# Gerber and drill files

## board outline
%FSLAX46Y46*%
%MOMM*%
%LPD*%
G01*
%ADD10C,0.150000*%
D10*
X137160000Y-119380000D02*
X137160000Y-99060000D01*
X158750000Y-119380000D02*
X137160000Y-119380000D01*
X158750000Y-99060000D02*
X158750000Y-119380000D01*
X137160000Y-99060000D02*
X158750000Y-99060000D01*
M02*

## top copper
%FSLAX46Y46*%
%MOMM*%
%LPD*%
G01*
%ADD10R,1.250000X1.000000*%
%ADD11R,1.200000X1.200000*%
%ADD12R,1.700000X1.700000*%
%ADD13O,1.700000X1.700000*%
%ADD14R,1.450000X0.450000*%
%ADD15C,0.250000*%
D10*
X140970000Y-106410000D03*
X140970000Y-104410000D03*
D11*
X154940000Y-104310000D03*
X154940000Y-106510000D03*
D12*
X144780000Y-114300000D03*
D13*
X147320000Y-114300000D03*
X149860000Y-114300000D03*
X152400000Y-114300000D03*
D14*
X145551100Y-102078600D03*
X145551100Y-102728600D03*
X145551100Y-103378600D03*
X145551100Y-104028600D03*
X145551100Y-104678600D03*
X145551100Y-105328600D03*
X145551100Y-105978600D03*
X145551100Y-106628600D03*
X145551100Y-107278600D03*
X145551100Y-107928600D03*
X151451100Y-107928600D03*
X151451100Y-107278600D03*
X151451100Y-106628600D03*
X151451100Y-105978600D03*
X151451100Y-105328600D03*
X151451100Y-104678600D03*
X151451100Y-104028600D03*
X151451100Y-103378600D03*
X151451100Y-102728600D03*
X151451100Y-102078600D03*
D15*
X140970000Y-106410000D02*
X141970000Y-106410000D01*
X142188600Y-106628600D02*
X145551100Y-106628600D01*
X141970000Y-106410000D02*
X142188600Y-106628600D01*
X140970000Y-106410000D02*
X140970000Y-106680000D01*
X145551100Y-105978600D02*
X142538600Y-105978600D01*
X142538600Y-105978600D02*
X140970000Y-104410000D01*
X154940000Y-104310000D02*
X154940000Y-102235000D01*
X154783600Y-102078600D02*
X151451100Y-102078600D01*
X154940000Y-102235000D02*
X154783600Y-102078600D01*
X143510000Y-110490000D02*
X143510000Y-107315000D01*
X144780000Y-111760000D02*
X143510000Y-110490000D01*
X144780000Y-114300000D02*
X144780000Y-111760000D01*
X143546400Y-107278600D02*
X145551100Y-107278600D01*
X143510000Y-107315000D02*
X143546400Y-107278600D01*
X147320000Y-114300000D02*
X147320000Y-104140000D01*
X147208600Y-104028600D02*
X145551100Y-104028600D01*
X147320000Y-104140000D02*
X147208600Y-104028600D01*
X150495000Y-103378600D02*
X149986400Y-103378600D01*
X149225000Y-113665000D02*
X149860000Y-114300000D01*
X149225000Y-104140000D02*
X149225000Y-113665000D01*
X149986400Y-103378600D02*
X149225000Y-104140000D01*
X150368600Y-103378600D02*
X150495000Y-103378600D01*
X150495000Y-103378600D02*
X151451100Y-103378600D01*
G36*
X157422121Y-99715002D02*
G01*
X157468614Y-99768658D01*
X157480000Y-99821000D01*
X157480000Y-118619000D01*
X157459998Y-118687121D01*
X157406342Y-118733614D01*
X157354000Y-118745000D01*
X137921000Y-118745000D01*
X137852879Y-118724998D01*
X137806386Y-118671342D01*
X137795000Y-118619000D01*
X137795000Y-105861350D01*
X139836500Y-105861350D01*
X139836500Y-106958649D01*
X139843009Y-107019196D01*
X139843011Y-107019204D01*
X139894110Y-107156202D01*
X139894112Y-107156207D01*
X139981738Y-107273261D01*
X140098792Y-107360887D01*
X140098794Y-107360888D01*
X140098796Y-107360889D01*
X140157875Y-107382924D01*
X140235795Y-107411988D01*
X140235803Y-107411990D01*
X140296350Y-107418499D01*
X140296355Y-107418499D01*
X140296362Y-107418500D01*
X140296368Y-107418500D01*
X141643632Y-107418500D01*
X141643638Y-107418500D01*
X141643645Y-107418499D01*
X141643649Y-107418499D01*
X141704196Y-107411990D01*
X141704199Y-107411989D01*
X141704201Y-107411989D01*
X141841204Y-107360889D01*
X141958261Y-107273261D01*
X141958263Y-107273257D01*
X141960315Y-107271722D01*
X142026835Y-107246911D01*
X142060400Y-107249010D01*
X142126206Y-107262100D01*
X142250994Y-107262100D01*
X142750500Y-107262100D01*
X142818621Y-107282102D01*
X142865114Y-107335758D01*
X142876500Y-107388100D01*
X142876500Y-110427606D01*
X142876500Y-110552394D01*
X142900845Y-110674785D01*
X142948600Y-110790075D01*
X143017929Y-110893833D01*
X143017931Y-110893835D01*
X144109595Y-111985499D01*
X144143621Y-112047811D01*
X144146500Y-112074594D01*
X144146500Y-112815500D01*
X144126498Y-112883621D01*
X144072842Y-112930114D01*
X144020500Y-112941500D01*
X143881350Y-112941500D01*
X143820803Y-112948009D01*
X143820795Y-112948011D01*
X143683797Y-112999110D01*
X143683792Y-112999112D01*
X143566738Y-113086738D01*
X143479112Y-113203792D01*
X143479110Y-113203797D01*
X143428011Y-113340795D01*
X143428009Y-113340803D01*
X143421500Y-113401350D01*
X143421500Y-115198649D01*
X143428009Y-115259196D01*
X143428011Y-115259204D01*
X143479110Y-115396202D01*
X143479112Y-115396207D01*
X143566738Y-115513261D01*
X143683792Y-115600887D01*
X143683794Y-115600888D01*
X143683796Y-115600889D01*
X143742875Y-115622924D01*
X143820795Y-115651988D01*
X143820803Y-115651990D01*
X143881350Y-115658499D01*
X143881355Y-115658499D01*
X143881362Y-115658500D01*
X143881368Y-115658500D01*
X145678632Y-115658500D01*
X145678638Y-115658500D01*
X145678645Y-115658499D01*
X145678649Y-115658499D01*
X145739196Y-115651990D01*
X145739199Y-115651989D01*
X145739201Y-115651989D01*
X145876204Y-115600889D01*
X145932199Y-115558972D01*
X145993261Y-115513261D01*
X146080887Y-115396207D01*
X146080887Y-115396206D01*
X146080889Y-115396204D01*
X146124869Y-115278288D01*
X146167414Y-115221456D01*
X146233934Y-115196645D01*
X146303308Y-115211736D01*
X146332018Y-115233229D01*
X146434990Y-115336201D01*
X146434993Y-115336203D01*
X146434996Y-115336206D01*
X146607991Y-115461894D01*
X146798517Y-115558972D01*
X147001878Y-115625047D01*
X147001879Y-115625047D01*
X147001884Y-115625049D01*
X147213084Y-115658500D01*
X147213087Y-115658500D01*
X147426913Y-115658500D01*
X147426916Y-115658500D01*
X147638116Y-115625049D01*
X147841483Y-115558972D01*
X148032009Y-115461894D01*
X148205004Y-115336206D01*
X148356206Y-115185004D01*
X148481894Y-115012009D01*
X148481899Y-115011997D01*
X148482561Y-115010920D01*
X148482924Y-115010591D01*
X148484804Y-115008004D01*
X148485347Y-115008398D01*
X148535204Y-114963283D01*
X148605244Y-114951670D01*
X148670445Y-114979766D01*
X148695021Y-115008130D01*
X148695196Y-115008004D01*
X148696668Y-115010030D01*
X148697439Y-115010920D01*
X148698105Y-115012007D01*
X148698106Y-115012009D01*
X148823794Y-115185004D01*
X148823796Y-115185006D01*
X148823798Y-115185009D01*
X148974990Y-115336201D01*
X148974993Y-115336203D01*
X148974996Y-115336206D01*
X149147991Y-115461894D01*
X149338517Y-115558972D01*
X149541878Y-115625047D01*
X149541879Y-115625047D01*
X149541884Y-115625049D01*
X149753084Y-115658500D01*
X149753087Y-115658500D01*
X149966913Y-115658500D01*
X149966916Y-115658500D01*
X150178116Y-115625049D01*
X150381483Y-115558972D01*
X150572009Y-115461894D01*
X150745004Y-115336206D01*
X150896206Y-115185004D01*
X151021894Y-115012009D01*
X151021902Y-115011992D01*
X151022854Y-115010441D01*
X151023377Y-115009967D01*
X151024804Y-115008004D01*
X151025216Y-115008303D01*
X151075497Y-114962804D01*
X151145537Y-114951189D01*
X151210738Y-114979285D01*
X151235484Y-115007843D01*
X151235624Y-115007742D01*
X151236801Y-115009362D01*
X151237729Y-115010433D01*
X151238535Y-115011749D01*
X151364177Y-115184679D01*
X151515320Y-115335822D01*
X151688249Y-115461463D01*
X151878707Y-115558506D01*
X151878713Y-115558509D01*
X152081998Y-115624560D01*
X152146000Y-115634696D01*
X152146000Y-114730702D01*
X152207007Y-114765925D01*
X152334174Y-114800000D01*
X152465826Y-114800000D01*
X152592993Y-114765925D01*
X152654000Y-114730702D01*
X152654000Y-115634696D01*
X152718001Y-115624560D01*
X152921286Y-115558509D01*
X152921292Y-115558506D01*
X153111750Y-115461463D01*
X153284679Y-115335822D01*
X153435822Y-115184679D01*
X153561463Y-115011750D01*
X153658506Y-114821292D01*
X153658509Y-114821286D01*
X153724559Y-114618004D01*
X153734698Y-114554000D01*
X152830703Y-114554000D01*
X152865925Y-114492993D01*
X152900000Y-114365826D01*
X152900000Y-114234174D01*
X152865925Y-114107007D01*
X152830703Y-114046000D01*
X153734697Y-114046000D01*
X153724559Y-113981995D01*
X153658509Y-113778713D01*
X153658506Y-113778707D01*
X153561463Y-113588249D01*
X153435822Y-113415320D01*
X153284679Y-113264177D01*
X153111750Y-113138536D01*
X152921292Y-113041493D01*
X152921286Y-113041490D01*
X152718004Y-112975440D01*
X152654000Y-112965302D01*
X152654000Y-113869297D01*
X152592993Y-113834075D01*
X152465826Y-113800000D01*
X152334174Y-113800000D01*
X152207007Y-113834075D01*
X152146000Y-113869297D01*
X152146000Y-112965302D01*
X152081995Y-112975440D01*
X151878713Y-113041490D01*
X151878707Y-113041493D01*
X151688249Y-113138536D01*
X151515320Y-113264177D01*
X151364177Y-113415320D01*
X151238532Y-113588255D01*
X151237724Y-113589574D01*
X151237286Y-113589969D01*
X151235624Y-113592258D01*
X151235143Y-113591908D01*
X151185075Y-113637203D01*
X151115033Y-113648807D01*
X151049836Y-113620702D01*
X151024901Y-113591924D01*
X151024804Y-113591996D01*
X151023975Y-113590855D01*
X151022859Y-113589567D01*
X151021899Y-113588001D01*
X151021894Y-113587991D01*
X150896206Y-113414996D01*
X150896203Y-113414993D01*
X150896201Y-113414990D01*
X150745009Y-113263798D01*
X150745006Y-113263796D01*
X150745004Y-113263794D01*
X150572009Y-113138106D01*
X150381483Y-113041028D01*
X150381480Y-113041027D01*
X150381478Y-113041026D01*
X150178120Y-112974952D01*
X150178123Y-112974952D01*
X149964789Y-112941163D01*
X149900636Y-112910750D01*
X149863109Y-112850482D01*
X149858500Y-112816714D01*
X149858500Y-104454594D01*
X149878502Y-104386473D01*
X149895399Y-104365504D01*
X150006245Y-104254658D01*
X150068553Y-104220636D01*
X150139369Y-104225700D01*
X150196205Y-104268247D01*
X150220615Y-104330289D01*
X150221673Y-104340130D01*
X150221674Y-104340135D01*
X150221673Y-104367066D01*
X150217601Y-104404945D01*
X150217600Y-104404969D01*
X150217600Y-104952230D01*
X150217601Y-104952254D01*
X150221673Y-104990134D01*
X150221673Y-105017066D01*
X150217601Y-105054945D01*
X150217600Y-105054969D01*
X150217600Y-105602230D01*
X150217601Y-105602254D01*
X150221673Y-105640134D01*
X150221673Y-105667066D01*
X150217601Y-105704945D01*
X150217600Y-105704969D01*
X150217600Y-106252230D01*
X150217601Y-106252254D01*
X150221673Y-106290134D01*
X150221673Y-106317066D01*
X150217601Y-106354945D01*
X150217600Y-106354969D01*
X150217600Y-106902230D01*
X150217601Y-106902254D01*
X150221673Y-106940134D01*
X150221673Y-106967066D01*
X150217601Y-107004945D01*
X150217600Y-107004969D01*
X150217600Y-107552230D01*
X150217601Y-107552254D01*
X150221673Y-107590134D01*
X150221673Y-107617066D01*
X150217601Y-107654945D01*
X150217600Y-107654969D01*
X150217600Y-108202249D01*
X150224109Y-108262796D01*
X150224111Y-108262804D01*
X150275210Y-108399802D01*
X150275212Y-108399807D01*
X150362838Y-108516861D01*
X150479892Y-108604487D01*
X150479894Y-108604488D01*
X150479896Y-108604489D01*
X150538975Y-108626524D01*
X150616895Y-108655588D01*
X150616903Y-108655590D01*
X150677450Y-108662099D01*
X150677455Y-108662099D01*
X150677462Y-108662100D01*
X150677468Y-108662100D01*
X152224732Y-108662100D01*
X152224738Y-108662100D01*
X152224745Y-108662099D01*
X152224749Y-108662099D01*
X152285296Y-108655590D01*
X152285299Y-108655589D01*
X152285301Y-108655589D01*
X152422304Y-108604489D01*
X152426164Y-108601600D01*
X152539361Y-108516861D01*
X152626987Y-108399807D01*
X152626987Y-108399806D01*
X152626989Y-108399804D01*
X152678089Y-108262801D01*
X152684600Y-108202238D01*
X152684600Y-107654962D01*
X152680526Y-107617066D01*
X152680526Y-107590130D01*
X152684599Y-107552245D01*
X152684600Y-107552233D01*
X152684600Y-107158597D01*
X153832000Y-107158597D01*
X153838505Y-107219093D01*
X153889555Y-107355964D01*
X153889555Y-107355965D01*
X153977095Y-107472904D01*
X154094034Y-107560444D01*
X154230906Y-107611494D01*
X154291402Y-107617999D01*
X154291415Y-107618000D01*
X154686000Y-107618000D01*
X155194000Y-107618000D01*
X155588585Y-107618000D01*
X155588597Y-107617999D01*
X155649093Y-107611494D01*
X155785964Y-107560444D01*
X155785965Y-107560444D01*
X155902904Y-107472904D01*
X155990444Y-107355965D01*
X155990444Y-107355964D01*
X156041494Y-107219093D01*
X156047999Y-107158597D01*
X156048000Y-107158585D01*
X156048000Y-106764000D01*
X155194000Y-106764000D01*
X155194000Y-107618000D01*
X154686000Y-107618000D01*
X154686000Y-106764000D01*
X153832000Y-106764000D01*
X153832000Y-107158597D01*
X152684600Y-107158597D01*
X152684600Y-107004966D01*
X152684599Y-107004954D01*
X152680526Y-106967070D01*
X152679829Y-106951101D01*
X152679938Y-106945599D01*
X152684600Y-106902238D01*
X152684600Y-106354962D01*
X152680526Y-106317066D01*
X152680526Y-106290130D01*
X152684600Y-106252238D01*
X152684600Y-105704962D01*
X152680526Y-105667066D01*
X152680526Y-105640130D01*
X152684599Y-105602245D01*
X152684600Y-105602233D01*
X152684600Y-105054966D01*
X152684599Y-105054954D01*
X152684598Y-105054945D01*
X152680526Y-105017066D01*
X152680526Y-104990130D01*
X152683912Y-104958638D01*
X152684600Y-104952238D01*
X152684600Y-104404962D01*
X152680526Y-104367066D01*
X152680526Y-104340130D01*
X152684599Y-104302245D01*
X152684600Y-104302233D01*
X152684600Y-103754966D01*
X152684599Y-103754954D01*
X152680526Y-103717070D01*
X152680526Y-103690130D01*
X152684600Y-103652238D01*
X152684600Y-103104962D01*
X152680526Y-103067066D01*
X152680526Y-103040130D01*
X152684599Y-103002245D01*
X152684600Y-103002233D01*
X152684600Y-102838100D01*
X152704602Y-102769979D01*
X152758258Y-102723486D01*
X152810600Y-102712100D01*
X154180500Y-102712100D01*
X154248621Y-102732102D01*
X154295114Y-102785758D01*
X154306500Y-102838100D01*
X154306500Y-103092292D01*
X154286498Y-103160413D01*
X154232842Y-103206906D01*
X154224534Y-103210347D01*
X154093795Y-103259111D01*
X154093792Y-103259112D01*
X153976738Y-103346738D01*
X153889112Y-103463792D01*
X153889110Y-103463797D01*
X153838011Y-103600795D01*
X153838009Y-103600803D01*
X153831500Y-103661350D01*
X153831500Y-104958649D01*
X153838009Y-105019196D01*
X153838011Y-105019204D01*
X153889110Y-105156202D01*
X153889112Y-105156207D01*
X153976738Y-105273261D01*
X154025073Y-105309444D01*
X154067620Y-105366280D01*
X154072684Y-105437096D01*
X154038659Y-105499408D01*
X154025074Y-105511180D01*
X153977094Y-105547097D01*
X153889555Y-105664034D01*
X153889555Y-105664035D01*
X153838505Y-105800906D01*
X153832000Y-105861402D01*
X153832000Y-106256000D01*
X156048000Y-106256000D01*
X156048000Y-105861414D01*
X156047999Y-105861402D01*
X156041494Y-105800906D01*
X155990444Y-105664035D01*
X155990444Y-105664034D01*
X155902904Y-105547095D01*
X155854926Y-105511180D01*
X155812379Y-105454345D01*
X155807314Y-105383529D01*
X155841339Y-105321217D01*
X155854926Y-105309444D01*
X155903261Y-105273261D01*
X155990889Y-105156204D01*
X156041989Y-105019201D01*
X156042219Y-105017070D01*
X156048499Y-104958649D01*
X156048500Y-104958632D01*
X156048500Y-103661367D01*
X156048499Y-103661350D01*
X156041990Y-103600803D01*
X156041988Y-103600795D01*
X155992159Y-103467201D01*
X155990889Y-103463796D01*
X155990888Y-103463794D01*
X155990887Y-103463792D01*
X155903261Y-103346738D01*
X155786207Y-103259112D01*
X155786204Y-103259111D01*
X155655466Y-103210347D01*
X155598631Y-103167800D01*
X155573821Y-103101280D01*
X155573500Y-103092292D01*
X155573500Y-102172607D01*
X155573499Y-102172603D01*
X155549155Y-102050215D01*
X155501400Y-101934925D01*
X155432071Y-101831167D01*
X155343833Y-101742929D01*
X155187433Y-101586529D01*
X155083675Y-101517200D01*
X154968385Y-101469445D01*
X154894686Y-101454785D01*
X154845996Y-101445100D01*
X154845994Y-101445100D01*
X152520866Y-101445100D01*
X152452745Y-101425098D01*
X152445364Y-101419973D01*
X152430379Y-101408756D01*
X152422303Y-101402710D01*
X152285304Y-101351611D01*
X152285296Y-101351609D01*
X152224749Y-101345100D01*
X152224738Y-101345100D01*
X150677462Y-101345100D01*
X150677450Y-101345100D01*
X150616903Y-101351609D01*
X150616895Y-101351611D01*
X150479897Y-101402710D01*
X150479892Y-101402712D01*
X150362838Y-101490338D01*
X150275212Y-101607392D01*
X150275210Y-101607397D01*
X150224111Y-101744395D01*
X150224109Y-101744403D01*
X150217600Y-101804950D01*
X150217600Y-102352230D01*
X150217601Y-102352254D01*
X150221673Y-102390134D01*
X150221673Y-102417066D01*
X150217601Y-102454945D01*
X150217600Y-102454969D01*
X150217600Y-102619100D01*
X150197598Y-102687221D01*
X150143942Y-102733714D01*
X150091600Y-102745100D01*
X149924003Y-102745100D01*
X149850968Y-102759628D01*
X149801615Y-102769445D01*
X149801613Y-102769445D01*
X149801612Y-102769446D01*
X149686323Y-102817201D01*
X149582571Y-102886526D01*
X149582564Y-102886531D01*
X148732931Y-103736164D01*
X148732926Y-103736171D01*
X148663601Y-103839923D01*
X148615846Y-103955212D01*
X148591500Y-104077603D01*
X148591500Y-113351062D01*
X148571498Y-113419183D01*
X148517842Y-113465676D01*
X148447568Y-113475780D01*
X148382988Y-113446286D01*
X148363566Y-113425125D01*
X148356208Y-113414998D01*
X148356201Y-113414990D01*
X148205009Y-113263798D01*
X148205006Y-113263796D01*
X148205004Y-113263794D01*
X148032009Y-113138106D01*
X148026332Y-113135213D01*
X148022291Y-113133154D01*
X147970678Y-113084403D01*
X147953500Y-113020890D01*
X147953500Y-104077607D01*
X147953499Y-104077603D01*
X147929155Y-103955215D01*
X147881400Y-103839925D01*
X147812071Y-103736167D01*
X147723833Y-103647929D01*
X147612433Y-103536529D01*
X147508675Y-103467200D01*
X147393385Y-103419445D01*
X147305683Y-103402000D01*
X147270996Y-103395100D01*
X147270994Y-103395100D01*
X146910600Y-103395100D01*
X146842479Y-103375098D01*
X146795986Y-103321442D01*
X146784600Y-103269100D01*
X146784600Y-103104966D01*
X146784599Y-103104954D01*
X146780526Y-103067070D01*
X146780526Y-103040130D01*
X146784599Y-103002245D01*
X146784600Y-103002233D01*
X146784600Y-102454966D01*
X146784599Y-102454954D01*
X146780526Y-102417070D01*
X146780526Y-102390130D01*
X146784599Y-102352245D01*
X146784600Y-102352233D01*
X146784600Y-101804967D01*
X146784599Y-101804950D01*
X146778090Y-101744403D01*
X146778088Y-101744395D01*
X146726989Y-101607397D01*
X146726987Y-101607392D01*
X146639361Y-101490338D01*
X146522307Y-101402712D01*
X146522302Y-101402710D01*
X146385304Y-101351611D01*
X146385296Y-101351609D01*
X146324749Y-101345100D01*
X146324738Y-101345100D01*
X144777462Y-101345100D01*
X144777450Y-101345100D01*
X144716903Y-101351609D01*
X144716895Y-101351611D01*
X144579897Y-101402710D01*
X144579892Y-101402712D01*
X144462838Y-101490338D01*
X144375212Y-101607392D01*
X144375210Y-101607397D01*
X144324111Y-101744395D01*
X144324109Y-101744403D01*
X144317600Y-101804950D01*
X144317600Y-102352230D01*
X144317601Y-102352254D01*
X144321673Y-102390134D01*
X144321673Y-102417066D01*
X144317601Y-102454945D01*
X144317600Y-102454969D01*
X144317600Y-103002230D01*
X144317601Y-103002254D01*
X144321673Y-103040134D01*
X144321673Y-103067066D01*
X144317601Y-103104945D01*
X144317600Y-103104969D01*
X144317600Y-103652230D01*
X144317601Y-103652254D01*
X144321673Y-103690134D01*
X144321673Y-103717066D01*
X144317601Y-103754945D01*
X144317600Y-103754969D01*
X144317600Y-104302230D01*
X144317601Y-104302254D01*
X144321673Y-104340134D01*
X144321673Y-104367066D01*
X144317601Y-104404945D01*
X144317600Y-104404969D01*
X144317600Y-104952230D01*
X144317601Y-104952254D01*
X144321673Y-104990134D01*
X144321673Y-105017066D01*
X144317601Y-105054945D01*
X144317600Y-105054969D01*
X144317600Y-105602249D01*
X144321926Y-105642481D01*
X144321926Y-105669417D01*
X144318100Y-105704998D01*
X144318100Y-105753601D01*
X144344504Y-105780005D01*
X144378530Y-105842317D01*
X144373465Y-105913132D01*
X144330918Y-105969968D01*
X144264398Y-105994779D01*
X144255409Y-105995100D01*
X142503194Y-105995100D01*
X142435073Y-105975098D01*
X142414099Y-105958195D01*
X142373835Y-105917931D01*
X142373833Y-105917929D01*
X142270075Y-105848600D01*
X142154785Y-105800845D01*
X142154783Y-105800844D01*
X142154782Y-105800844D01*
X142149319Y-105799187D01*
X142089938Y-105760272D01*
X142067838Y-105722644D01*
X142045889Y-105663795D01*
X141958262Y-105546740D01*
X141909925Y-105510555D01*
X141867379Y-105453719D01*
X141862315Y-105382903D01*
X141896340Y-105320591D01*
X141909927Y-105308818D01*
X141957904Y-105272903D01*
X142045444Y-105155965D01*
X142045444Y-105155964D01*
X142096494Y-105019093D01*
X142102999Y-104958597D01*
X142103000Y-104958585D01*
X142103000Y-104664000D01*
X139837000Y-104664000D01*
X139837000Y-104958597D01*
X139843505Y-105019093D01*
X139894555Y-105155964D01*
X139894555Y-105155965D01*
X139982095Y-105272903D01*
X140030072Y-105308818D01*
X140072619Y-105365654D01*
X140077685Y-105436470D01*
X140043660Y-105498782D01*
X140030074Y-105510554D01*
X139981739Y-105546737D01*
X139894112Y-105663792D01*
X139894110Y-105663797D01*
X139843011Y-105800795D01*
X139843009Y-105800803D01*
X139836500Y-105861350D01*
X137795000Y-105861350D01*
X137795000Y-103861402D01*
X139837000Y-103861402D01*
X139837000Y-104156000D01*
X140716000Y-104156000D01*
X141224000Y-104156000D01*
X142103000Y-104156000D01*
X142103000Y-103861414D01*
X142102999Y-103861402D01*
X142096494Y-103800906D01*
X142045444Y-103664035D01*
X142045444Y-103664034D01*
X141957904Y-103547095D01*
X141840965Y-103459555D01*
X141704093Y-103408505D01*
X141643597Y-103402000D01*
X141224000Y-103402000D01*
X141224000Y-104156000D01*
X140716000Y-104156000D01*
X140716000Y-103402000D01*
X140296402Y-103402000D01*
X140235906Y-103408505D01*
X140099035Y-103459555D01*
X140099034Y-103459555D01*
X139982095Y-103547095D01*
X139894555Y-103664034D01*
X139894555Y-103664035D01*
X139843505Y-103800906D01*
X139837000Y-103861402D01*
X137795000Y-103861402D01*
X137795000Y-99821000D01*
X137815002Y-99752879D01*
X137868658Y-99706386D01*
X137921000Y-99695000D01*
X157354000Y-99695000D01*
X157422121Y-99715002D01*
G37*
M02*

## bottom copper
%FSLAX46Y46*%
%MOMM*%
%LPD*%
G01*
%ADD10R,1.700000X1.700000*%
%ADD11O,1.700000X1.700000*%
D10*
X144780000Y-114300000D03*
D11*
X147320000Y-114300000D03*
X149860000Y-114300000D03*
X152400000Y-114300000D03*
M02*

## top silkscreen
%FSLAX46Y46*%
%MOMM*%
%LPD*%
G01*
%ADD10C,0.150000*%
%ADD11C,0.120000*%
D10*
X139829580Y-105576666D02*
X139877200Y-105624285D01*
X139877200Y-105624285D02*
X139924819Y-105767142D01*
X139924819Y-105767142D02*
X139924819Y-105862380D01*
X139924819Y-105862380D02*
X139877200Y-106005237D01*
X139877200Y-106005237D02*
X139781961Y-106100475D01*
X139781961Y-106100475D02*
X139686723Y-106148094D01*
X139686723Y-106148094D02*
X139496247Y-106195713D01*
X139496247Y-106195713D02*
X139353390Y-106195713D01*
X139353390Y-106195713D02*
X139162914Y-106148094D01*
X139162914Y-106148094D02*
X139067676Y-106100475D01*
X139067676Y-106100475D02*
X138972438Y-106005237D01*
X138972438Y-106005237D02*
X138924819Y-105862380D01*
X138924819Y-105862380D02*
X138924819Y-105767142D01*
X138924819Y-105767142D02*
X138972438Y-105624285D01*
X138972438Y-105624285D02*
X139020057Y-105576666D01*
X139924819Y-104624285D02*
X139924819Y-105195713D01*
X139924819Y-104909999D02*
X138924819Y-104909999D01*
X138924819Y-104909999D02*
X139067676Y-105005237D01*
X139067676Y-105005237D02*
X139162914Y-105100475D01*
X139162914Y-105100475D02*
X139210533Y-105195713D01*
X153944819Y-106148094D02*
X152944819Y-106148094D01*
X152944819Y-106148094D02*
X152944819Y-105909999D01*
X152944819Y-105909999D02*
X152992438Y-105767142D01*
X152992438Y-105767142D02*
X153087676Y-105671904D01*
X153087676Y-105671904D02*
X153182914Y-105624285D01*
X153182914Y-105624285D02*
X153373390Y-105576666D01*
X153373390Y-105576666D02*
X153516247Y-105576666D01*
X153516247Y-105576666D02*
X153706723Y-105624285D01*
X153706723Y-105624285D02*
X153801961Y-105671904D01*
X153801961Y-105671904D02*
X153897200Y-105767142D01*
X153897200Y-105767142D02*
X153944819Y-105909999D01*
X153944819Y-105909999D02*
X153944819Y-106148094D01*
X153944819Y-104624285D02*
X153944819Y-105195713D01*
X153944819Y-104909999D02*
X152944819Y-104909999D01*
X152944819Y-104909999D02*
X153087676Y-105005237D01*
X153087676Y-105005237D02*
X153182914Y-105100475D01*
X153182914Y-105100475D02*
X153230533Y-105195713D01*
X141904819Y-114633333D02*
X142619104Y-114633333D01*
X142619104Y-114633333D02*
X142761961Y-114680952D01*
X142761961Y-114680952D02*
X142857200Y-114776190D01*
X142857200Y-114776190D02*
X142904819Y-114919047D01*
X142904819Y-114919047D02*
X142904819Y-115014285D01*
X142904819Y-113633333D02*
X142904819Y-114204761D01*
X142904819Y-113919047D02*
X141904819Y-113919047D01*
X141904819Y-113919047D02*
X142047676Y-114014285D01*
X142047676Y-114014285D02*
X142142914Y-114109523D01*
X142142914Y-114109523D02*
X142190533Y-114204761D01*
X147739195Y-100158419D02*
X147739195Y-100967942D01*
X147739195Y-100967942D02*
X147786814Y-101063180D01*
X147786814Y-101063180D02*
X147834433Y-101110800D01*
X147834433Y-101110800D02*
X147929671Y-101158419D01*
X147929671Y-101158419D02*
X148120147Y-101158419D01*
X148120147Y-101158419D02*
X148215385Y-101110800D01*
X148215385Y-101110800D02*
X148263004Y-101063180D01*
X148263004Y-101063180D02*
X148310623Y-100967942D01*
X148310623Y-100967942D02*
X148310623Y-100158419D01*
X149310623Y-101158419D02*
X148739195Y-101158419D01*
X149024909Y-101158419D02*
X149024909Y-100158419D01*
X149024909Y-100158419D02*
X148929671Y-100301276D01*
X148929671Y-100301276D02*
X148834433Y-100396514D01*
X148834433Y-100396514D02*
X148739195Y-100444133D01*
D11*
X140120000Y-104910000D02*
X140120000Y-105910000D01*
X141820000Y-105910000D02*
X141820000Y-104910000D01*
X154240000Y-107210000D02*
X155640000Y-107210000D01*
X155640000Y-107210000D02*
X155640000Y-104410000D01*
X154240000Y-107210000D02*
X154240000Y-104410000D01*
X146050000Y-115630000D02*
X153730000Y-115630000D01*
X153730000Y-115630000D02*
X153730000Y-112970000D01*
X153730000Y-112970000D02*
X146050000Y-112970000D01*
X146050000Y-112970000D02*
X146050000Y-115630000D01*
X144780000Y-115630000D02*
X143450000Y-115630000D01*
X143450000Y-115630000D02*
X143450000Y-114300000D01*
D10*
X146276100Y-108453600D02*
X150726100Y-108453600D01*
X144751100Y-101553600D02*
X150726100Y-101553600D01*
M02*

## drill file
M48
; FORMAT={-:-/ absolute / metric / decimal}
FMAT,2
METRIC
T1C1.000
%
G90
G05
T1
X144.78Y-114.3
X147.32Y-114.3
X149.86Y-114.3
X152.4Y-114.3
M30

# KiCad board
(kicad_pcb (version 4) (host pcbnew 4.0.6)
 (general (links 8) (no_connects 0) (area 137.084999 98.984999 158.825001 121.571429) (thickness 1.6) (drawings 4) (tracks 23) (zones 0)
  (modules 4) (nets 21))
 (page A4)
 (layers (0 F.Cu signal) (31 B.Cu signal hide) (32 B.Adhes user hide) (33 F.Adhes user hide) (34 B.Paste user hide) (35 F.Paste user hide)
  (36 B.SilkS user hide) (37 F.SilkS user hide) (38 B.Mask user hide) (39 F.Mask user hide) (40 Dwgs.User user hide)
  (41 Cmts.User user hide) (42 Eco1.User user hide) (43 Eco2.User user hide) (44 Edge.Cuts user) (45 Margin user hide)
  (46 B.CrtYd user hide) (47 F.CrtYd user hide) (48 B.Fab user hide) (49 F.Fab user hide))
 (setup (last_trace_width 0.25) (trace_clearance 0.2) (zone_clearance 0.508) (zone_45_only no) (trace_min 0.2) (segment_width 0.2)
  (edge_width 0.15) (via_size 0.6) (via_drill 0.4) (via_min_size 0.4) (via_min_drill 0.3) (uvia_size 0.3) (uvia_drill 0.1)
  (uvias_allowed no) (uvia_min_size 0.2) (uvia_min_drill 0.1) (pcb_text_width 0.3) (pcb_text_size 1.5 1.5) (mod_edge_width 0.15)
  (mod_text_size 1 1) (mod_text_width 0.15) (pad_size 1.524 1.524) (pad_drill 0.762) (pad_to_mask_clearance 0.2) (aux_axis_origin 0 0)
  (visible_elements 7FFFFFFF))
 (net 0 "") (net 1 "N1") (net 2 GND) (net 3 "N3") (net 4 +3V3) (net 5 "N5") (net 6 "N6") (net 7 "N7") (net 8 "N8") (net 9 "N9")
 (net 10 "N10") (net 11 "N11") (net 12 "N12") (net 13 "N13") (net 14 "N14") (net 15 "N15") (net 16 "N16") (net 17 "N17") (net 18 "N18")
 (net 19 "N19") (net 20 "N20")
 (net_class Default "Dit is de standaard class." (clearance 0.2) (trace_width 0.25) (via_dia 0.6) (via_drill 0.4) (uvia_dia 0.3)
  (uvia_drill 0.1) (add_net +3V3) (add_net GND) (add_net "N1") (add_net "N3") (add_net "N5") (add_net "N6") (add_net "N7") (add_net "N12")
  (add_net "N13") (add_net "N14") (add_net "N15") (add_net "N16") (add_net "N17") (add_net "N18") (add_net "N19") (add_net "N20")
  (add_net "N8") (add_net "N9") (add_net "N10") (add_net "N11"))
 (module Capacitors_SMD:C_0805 (layer F.Cu) (at 140.97 105.41 90)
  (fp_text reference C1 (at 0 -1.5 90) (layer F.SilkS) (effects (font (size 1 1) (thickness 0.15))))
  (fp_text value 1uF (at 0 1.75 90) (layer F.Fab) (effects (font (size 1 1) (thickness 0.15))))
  (fp_line (start 0.5 -0.85) (end -0.5 -0.85) (layer F.SilkS) (width 0.12))
  (fp_line (start -0.5 0.85) (end 0.5 0.85) (layer F.SilkS) (width 0.12))
  (pad 1 smd rect (at -1 0 90) (size 1 1.25) (layers F.Cu F.Paste F.Mask) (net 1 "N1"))
  (pad 2 smd rect (at 1 0 90) (size 1 1.25) (layers F.Cu F.Paste F.Mask) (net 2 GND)))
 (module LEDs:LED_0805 (layer F.Cu) (at 154.94 105.41 90)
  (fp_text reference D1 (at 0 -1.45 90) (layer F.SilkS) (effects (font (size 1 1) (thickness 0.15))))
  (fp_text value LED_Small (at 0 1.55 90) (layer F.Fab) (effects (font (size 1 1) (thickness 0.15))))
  (fp_line (start -1.8 -0.7) (end -1.8 0.7) (layer F.SilkS) (width 0.12))
  (fp_line (start -1.8 0.7) (end 1 0.7) (layer F.SilkS) (width 0.12))
  (fp_line (start -1.8 -0.7) (end 1 -0.7) (layer F.SilkS) (width 0.12))
  (pad 2 smd rect (at 1.1 0 270) (size 1.2 1.2) (layers F.Cu F.Paste F.Mask) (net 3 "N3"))
  (pad 1 smd rect (at -1.1 0 270) (size 1.2 1.2) (layers F.Cu F.Paste F.Mask) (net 2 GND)))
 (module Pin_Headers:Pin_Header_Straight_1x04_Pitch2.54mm (layer F.Cu) (at 144.78 114.3 90)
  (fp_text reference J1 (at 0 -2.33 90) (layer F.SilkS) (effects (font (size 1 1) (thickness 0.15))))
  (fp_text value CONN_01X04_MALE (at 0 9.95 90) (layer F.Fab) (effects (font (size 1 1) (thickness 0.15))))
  (fp_line (start -1.33 1.27) (end -1.33 8.95) (layer F.SilkS) (width 0.12))
  (fp_line (start -1.33 8.95) (end 1.33 8.95) (layer F.SilkS) (width 0.12))
  (fp_line (start 1.33 8.95) (end 1.33 1.27) (layer F.SilkS) (width 0.12))
  (fp_line (start 1.33 1.27) (end -1.33 1.27) (layer F.SilkS) (width 0.12))
  (fp_line (start -1.33 0) (end -1.33 -1.33) (layer F.SilkS) (width 0.12))
  (fp_line (start -1.33 -1.33) (end 0 -1.33) (layer F.SilkS) (width 0.12))
  (pad 1 thru_hole rect (at 0 0 90) (size 1.7 1.7) (drill 1) (layers *.Cu *.Mask) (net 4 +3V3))
  (pad 2 thru_hole oval (at 0 2.54 90) (size 1.7 1.7) (drill 1) (layers *.Cu *.Mask) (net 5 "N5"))
  (pad 3 thru_hole oval (at 0 5.08 90) (size 1.7 1.7) (drill 1) (layers *.Cu *.Mask) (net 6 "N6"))
  (pad 4 thru_hole oval (at 0 7.62 90) (size 1.7 1.7) (drill 1) (layers *.Cu *.Mask) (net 2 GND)))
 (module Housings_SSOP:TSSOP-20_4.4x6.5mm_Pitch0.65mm (layer F.Cu) (at 148.5011 105.0036)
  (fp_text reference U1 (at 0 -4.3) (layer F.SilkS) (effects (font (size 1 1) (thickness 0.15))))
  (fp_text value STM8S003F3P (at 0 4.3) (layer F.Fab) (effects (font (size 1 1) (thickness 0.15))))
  (fp_line (start -2.225 3.45) (end 2.225 3.45) (layer F.SilkS) (width 0.15))
  (fp_line (start -3.75 -3.45) (end 2.225 -3.45) (layer F.SilkS) (width 0.15))
  (pad 1 smd rect (at -2.95 -2.925) (size 1.45 0.45) (layers F.Cu F.Paste F.Mask) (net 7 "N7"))
  (pad 2 smd rect (at -2.95 -2.275) (size 1.45 0.45) (layers F.Cu F.Paste F.Mask) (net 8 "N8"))
  (pad 3 smd rect (at -2.95 -1.625) (size 1.45 0.45) (layers F.Cu F.Paste F.Mask) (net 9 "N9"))
  (pad 4 smd rect (at -2.95 -0.975) (size 1.45 0.45) (layers F.Cu F.Paste F.Mask) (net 5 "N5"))
  (pad 5 smd rect (at -2.95 -0.325) (size 1.45 0.45) (layers F.Cu F.Paste F.Mask) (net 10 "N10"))
  (pad 6 smd rect (at -2.95 0.325) (size 1.45 0.45) (layers F.Cu F.Paste F.Mask) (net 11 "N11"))
  (pad 7 smd rect (at -2.95 0.975) (size 1.45 0.45) (layers F.Cu F.Paste F.Mask) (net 2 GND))
  (pad 8 smd rect (at -2.95 1.625) (size 1.45 0.45) (layers F.Cu F.Paste F.Mask) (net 1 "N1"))
  (pad 9 smd rect (at -2.95 2.275) (size 1.45 0.45) (layers F.Cu F.Paste F.Mask) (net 4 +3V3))
  (pad 10 smd rect (at -2.95 2.925) (size 1.45 0.45) (layers F.Cu F.Paste F.Mask) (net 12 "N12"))
  (pad 11 smd rect (at 2.95 2.925) (size 1.45 0.45) (layers F.Cu F.Paste F.Mask) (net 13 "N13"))
  (pad 12 smd rect (at 2.95 2.275) (size 1.45 0.45) (layers F.Cu F.Paste F.Mask) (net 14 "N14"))
  (pad 13 smd rect (at 2.95 1.625) (size 1.45 0.45) (layers F.Cu F.Paste F.Mask) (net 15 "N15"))
  (pad 14 smd rect (at 2.95 0.975) (size 1.45 0.45) (layers F.Cu F.Paste F.Mask) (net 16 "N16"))
  (pad 15 smd rect (at 2.95 0.325) (size 1.45 0.45) (layers F.Cu F.Paste F.Mask) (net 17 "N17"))
  (pad 16 smd rect (at 2.95 -0.325) (size 1.45 0.45) (layers F.Cu F.Paste F.Mask) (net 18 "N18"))
  (pad 17 smd rect (at 2.95 -0.975) (size 1.45 0.45) (layers F.Cu F.Paste F.Mask) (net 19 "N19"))
  (pad 18 smd rect (at 2.95 -1.625) (size 1.45 0.45) (layers F.Cu F.Paste F.Mask) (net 6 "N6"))
  (pad 19 smd rect (at 2.95 -2.275) (size 1.45 0.45) (layers F.Cu F.Paste F.Mask) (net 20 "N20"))
  (pad 20 smd rect (at 2.95 -2.925) (size 1.45 0.45) (layers F.Cu F.Paste F.Mask) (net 3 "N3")))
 (gr_line (start 137.16 119.38) (end 137.16 99.06) (angle 90) (layer Edge.Cuts) (width 0.15))
 (gr_line (start 158.75 119.38) (end 137.16 119.38) (angle 90) (layer Edge.Cuts) (width 0.15))
 (gr_line (start 158.75 99.06) (end 158.75 119.38) (angle 90) (layer Edge.Cuts) (width 0.15))
 (gr_line (start 137.16 99.06) (end 158.75 99.06) (angle 90) (layer Edge.Cuts) (width 0.15))
 (segment (start 140.97 106.41) (end 141.97 106.41) (width 0.25) (layer F.Cu) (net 1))
 (segment (start 142.1886 106.6286) (end 145.5511 106.6286) (width 0.25) (layer F.Cu) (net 1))
 (segment (start 141.97 106.41) (end 142.1886 106.6286) (width 0.25) (layer F.Cu) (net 1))
 (segment (start 140.97 106.41) (end 140.97 106.68) (width 0.25) (layer F.Cu) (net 1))
 (segment (start 145.5511 105.9786) (end 142.5386 105.9786) (width 0.25) (layer F.Cu) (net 2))
 (segment (start 142.5386 105.9786) (end 140.97 104.41) (width 0.25) (layer F.Cu) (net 2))
 (segment (start 154.94 104.31) (end 154.94 102.235) (width 0.25) (layer F.Cu) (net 3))
 (segment (start 154.7836 102.0786) (end 151.4511 102.0786) (width 0.25) (layer F.Cu) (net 3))
 (segment (start 154.94 102.235) (end 154.7836 102.0786) (width 0.25) (layer F.Cu) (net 3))
 (segment (start 143.51 110.49) (end 143.51 107.315) (width 0.25) (layer F.Cu) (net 4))
 (segment (start 144.78 111.76) (end 143.51 110.49) (width 0.25) (layer F.Cu) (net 4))
 (segment (start 144.78 114.3) (end 144.78 111.76) (width 0.25) (layer F.Cu) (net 4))
 (segment (start 143.5464 107.2786) (end 145.5511 107.2786) (width 0.25) (layer F.Cu) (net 4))
 (segment (start 143.51 107.315) (end 143.5464 107.2786) (width 0.25) (layer F.Cu) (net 4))
 (segment (start 147.32 114.3) (end 147.32 104.14) (width 0.25) (layer F.Cu) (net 5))
 (segment (start 147.2086 104.0286) (end 145.5511 104.0286) (width 0.25) (layer F.Cu) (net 5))
 (segment (start 147.32 104.14) (end 147.2086 104.0286) (width 0.25) (layer F.Cu) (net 5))
 (segment (start 150.495 103.3786) (end 149.9864 103.3786) (width 0.25) (layer F.Cu) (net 6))
 (segment (start 149.225 113.665) (end 149.86 114.3) (width 0.25) (layer F.Cu) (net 6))
 (segment (start 149.225 104.14) (end 149.225 113.665) (width 0.25) (layer F.Cu) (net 6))
 (segment (start 149.9864 103.3786) (end 149.225 104.14) (width 0.25) (layer F.Cu) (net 6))
 (segment (start 150.3686 103.3786) (end 150.495 103.3786) (width 0.25) (layer F.Cu) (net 6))
 (segment (start 150.495 103.3786) (end 151.4511 103.3786) (width 0.25) (layer F.Cu) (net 6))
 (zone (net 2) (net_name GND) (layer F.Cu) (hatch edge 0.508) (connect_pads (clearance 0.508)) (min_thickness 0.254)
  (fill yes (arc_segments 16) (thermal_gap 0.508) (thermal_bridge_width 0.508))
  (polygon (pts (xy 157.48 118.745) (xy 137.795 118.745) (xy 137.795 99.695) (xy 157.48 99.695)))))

